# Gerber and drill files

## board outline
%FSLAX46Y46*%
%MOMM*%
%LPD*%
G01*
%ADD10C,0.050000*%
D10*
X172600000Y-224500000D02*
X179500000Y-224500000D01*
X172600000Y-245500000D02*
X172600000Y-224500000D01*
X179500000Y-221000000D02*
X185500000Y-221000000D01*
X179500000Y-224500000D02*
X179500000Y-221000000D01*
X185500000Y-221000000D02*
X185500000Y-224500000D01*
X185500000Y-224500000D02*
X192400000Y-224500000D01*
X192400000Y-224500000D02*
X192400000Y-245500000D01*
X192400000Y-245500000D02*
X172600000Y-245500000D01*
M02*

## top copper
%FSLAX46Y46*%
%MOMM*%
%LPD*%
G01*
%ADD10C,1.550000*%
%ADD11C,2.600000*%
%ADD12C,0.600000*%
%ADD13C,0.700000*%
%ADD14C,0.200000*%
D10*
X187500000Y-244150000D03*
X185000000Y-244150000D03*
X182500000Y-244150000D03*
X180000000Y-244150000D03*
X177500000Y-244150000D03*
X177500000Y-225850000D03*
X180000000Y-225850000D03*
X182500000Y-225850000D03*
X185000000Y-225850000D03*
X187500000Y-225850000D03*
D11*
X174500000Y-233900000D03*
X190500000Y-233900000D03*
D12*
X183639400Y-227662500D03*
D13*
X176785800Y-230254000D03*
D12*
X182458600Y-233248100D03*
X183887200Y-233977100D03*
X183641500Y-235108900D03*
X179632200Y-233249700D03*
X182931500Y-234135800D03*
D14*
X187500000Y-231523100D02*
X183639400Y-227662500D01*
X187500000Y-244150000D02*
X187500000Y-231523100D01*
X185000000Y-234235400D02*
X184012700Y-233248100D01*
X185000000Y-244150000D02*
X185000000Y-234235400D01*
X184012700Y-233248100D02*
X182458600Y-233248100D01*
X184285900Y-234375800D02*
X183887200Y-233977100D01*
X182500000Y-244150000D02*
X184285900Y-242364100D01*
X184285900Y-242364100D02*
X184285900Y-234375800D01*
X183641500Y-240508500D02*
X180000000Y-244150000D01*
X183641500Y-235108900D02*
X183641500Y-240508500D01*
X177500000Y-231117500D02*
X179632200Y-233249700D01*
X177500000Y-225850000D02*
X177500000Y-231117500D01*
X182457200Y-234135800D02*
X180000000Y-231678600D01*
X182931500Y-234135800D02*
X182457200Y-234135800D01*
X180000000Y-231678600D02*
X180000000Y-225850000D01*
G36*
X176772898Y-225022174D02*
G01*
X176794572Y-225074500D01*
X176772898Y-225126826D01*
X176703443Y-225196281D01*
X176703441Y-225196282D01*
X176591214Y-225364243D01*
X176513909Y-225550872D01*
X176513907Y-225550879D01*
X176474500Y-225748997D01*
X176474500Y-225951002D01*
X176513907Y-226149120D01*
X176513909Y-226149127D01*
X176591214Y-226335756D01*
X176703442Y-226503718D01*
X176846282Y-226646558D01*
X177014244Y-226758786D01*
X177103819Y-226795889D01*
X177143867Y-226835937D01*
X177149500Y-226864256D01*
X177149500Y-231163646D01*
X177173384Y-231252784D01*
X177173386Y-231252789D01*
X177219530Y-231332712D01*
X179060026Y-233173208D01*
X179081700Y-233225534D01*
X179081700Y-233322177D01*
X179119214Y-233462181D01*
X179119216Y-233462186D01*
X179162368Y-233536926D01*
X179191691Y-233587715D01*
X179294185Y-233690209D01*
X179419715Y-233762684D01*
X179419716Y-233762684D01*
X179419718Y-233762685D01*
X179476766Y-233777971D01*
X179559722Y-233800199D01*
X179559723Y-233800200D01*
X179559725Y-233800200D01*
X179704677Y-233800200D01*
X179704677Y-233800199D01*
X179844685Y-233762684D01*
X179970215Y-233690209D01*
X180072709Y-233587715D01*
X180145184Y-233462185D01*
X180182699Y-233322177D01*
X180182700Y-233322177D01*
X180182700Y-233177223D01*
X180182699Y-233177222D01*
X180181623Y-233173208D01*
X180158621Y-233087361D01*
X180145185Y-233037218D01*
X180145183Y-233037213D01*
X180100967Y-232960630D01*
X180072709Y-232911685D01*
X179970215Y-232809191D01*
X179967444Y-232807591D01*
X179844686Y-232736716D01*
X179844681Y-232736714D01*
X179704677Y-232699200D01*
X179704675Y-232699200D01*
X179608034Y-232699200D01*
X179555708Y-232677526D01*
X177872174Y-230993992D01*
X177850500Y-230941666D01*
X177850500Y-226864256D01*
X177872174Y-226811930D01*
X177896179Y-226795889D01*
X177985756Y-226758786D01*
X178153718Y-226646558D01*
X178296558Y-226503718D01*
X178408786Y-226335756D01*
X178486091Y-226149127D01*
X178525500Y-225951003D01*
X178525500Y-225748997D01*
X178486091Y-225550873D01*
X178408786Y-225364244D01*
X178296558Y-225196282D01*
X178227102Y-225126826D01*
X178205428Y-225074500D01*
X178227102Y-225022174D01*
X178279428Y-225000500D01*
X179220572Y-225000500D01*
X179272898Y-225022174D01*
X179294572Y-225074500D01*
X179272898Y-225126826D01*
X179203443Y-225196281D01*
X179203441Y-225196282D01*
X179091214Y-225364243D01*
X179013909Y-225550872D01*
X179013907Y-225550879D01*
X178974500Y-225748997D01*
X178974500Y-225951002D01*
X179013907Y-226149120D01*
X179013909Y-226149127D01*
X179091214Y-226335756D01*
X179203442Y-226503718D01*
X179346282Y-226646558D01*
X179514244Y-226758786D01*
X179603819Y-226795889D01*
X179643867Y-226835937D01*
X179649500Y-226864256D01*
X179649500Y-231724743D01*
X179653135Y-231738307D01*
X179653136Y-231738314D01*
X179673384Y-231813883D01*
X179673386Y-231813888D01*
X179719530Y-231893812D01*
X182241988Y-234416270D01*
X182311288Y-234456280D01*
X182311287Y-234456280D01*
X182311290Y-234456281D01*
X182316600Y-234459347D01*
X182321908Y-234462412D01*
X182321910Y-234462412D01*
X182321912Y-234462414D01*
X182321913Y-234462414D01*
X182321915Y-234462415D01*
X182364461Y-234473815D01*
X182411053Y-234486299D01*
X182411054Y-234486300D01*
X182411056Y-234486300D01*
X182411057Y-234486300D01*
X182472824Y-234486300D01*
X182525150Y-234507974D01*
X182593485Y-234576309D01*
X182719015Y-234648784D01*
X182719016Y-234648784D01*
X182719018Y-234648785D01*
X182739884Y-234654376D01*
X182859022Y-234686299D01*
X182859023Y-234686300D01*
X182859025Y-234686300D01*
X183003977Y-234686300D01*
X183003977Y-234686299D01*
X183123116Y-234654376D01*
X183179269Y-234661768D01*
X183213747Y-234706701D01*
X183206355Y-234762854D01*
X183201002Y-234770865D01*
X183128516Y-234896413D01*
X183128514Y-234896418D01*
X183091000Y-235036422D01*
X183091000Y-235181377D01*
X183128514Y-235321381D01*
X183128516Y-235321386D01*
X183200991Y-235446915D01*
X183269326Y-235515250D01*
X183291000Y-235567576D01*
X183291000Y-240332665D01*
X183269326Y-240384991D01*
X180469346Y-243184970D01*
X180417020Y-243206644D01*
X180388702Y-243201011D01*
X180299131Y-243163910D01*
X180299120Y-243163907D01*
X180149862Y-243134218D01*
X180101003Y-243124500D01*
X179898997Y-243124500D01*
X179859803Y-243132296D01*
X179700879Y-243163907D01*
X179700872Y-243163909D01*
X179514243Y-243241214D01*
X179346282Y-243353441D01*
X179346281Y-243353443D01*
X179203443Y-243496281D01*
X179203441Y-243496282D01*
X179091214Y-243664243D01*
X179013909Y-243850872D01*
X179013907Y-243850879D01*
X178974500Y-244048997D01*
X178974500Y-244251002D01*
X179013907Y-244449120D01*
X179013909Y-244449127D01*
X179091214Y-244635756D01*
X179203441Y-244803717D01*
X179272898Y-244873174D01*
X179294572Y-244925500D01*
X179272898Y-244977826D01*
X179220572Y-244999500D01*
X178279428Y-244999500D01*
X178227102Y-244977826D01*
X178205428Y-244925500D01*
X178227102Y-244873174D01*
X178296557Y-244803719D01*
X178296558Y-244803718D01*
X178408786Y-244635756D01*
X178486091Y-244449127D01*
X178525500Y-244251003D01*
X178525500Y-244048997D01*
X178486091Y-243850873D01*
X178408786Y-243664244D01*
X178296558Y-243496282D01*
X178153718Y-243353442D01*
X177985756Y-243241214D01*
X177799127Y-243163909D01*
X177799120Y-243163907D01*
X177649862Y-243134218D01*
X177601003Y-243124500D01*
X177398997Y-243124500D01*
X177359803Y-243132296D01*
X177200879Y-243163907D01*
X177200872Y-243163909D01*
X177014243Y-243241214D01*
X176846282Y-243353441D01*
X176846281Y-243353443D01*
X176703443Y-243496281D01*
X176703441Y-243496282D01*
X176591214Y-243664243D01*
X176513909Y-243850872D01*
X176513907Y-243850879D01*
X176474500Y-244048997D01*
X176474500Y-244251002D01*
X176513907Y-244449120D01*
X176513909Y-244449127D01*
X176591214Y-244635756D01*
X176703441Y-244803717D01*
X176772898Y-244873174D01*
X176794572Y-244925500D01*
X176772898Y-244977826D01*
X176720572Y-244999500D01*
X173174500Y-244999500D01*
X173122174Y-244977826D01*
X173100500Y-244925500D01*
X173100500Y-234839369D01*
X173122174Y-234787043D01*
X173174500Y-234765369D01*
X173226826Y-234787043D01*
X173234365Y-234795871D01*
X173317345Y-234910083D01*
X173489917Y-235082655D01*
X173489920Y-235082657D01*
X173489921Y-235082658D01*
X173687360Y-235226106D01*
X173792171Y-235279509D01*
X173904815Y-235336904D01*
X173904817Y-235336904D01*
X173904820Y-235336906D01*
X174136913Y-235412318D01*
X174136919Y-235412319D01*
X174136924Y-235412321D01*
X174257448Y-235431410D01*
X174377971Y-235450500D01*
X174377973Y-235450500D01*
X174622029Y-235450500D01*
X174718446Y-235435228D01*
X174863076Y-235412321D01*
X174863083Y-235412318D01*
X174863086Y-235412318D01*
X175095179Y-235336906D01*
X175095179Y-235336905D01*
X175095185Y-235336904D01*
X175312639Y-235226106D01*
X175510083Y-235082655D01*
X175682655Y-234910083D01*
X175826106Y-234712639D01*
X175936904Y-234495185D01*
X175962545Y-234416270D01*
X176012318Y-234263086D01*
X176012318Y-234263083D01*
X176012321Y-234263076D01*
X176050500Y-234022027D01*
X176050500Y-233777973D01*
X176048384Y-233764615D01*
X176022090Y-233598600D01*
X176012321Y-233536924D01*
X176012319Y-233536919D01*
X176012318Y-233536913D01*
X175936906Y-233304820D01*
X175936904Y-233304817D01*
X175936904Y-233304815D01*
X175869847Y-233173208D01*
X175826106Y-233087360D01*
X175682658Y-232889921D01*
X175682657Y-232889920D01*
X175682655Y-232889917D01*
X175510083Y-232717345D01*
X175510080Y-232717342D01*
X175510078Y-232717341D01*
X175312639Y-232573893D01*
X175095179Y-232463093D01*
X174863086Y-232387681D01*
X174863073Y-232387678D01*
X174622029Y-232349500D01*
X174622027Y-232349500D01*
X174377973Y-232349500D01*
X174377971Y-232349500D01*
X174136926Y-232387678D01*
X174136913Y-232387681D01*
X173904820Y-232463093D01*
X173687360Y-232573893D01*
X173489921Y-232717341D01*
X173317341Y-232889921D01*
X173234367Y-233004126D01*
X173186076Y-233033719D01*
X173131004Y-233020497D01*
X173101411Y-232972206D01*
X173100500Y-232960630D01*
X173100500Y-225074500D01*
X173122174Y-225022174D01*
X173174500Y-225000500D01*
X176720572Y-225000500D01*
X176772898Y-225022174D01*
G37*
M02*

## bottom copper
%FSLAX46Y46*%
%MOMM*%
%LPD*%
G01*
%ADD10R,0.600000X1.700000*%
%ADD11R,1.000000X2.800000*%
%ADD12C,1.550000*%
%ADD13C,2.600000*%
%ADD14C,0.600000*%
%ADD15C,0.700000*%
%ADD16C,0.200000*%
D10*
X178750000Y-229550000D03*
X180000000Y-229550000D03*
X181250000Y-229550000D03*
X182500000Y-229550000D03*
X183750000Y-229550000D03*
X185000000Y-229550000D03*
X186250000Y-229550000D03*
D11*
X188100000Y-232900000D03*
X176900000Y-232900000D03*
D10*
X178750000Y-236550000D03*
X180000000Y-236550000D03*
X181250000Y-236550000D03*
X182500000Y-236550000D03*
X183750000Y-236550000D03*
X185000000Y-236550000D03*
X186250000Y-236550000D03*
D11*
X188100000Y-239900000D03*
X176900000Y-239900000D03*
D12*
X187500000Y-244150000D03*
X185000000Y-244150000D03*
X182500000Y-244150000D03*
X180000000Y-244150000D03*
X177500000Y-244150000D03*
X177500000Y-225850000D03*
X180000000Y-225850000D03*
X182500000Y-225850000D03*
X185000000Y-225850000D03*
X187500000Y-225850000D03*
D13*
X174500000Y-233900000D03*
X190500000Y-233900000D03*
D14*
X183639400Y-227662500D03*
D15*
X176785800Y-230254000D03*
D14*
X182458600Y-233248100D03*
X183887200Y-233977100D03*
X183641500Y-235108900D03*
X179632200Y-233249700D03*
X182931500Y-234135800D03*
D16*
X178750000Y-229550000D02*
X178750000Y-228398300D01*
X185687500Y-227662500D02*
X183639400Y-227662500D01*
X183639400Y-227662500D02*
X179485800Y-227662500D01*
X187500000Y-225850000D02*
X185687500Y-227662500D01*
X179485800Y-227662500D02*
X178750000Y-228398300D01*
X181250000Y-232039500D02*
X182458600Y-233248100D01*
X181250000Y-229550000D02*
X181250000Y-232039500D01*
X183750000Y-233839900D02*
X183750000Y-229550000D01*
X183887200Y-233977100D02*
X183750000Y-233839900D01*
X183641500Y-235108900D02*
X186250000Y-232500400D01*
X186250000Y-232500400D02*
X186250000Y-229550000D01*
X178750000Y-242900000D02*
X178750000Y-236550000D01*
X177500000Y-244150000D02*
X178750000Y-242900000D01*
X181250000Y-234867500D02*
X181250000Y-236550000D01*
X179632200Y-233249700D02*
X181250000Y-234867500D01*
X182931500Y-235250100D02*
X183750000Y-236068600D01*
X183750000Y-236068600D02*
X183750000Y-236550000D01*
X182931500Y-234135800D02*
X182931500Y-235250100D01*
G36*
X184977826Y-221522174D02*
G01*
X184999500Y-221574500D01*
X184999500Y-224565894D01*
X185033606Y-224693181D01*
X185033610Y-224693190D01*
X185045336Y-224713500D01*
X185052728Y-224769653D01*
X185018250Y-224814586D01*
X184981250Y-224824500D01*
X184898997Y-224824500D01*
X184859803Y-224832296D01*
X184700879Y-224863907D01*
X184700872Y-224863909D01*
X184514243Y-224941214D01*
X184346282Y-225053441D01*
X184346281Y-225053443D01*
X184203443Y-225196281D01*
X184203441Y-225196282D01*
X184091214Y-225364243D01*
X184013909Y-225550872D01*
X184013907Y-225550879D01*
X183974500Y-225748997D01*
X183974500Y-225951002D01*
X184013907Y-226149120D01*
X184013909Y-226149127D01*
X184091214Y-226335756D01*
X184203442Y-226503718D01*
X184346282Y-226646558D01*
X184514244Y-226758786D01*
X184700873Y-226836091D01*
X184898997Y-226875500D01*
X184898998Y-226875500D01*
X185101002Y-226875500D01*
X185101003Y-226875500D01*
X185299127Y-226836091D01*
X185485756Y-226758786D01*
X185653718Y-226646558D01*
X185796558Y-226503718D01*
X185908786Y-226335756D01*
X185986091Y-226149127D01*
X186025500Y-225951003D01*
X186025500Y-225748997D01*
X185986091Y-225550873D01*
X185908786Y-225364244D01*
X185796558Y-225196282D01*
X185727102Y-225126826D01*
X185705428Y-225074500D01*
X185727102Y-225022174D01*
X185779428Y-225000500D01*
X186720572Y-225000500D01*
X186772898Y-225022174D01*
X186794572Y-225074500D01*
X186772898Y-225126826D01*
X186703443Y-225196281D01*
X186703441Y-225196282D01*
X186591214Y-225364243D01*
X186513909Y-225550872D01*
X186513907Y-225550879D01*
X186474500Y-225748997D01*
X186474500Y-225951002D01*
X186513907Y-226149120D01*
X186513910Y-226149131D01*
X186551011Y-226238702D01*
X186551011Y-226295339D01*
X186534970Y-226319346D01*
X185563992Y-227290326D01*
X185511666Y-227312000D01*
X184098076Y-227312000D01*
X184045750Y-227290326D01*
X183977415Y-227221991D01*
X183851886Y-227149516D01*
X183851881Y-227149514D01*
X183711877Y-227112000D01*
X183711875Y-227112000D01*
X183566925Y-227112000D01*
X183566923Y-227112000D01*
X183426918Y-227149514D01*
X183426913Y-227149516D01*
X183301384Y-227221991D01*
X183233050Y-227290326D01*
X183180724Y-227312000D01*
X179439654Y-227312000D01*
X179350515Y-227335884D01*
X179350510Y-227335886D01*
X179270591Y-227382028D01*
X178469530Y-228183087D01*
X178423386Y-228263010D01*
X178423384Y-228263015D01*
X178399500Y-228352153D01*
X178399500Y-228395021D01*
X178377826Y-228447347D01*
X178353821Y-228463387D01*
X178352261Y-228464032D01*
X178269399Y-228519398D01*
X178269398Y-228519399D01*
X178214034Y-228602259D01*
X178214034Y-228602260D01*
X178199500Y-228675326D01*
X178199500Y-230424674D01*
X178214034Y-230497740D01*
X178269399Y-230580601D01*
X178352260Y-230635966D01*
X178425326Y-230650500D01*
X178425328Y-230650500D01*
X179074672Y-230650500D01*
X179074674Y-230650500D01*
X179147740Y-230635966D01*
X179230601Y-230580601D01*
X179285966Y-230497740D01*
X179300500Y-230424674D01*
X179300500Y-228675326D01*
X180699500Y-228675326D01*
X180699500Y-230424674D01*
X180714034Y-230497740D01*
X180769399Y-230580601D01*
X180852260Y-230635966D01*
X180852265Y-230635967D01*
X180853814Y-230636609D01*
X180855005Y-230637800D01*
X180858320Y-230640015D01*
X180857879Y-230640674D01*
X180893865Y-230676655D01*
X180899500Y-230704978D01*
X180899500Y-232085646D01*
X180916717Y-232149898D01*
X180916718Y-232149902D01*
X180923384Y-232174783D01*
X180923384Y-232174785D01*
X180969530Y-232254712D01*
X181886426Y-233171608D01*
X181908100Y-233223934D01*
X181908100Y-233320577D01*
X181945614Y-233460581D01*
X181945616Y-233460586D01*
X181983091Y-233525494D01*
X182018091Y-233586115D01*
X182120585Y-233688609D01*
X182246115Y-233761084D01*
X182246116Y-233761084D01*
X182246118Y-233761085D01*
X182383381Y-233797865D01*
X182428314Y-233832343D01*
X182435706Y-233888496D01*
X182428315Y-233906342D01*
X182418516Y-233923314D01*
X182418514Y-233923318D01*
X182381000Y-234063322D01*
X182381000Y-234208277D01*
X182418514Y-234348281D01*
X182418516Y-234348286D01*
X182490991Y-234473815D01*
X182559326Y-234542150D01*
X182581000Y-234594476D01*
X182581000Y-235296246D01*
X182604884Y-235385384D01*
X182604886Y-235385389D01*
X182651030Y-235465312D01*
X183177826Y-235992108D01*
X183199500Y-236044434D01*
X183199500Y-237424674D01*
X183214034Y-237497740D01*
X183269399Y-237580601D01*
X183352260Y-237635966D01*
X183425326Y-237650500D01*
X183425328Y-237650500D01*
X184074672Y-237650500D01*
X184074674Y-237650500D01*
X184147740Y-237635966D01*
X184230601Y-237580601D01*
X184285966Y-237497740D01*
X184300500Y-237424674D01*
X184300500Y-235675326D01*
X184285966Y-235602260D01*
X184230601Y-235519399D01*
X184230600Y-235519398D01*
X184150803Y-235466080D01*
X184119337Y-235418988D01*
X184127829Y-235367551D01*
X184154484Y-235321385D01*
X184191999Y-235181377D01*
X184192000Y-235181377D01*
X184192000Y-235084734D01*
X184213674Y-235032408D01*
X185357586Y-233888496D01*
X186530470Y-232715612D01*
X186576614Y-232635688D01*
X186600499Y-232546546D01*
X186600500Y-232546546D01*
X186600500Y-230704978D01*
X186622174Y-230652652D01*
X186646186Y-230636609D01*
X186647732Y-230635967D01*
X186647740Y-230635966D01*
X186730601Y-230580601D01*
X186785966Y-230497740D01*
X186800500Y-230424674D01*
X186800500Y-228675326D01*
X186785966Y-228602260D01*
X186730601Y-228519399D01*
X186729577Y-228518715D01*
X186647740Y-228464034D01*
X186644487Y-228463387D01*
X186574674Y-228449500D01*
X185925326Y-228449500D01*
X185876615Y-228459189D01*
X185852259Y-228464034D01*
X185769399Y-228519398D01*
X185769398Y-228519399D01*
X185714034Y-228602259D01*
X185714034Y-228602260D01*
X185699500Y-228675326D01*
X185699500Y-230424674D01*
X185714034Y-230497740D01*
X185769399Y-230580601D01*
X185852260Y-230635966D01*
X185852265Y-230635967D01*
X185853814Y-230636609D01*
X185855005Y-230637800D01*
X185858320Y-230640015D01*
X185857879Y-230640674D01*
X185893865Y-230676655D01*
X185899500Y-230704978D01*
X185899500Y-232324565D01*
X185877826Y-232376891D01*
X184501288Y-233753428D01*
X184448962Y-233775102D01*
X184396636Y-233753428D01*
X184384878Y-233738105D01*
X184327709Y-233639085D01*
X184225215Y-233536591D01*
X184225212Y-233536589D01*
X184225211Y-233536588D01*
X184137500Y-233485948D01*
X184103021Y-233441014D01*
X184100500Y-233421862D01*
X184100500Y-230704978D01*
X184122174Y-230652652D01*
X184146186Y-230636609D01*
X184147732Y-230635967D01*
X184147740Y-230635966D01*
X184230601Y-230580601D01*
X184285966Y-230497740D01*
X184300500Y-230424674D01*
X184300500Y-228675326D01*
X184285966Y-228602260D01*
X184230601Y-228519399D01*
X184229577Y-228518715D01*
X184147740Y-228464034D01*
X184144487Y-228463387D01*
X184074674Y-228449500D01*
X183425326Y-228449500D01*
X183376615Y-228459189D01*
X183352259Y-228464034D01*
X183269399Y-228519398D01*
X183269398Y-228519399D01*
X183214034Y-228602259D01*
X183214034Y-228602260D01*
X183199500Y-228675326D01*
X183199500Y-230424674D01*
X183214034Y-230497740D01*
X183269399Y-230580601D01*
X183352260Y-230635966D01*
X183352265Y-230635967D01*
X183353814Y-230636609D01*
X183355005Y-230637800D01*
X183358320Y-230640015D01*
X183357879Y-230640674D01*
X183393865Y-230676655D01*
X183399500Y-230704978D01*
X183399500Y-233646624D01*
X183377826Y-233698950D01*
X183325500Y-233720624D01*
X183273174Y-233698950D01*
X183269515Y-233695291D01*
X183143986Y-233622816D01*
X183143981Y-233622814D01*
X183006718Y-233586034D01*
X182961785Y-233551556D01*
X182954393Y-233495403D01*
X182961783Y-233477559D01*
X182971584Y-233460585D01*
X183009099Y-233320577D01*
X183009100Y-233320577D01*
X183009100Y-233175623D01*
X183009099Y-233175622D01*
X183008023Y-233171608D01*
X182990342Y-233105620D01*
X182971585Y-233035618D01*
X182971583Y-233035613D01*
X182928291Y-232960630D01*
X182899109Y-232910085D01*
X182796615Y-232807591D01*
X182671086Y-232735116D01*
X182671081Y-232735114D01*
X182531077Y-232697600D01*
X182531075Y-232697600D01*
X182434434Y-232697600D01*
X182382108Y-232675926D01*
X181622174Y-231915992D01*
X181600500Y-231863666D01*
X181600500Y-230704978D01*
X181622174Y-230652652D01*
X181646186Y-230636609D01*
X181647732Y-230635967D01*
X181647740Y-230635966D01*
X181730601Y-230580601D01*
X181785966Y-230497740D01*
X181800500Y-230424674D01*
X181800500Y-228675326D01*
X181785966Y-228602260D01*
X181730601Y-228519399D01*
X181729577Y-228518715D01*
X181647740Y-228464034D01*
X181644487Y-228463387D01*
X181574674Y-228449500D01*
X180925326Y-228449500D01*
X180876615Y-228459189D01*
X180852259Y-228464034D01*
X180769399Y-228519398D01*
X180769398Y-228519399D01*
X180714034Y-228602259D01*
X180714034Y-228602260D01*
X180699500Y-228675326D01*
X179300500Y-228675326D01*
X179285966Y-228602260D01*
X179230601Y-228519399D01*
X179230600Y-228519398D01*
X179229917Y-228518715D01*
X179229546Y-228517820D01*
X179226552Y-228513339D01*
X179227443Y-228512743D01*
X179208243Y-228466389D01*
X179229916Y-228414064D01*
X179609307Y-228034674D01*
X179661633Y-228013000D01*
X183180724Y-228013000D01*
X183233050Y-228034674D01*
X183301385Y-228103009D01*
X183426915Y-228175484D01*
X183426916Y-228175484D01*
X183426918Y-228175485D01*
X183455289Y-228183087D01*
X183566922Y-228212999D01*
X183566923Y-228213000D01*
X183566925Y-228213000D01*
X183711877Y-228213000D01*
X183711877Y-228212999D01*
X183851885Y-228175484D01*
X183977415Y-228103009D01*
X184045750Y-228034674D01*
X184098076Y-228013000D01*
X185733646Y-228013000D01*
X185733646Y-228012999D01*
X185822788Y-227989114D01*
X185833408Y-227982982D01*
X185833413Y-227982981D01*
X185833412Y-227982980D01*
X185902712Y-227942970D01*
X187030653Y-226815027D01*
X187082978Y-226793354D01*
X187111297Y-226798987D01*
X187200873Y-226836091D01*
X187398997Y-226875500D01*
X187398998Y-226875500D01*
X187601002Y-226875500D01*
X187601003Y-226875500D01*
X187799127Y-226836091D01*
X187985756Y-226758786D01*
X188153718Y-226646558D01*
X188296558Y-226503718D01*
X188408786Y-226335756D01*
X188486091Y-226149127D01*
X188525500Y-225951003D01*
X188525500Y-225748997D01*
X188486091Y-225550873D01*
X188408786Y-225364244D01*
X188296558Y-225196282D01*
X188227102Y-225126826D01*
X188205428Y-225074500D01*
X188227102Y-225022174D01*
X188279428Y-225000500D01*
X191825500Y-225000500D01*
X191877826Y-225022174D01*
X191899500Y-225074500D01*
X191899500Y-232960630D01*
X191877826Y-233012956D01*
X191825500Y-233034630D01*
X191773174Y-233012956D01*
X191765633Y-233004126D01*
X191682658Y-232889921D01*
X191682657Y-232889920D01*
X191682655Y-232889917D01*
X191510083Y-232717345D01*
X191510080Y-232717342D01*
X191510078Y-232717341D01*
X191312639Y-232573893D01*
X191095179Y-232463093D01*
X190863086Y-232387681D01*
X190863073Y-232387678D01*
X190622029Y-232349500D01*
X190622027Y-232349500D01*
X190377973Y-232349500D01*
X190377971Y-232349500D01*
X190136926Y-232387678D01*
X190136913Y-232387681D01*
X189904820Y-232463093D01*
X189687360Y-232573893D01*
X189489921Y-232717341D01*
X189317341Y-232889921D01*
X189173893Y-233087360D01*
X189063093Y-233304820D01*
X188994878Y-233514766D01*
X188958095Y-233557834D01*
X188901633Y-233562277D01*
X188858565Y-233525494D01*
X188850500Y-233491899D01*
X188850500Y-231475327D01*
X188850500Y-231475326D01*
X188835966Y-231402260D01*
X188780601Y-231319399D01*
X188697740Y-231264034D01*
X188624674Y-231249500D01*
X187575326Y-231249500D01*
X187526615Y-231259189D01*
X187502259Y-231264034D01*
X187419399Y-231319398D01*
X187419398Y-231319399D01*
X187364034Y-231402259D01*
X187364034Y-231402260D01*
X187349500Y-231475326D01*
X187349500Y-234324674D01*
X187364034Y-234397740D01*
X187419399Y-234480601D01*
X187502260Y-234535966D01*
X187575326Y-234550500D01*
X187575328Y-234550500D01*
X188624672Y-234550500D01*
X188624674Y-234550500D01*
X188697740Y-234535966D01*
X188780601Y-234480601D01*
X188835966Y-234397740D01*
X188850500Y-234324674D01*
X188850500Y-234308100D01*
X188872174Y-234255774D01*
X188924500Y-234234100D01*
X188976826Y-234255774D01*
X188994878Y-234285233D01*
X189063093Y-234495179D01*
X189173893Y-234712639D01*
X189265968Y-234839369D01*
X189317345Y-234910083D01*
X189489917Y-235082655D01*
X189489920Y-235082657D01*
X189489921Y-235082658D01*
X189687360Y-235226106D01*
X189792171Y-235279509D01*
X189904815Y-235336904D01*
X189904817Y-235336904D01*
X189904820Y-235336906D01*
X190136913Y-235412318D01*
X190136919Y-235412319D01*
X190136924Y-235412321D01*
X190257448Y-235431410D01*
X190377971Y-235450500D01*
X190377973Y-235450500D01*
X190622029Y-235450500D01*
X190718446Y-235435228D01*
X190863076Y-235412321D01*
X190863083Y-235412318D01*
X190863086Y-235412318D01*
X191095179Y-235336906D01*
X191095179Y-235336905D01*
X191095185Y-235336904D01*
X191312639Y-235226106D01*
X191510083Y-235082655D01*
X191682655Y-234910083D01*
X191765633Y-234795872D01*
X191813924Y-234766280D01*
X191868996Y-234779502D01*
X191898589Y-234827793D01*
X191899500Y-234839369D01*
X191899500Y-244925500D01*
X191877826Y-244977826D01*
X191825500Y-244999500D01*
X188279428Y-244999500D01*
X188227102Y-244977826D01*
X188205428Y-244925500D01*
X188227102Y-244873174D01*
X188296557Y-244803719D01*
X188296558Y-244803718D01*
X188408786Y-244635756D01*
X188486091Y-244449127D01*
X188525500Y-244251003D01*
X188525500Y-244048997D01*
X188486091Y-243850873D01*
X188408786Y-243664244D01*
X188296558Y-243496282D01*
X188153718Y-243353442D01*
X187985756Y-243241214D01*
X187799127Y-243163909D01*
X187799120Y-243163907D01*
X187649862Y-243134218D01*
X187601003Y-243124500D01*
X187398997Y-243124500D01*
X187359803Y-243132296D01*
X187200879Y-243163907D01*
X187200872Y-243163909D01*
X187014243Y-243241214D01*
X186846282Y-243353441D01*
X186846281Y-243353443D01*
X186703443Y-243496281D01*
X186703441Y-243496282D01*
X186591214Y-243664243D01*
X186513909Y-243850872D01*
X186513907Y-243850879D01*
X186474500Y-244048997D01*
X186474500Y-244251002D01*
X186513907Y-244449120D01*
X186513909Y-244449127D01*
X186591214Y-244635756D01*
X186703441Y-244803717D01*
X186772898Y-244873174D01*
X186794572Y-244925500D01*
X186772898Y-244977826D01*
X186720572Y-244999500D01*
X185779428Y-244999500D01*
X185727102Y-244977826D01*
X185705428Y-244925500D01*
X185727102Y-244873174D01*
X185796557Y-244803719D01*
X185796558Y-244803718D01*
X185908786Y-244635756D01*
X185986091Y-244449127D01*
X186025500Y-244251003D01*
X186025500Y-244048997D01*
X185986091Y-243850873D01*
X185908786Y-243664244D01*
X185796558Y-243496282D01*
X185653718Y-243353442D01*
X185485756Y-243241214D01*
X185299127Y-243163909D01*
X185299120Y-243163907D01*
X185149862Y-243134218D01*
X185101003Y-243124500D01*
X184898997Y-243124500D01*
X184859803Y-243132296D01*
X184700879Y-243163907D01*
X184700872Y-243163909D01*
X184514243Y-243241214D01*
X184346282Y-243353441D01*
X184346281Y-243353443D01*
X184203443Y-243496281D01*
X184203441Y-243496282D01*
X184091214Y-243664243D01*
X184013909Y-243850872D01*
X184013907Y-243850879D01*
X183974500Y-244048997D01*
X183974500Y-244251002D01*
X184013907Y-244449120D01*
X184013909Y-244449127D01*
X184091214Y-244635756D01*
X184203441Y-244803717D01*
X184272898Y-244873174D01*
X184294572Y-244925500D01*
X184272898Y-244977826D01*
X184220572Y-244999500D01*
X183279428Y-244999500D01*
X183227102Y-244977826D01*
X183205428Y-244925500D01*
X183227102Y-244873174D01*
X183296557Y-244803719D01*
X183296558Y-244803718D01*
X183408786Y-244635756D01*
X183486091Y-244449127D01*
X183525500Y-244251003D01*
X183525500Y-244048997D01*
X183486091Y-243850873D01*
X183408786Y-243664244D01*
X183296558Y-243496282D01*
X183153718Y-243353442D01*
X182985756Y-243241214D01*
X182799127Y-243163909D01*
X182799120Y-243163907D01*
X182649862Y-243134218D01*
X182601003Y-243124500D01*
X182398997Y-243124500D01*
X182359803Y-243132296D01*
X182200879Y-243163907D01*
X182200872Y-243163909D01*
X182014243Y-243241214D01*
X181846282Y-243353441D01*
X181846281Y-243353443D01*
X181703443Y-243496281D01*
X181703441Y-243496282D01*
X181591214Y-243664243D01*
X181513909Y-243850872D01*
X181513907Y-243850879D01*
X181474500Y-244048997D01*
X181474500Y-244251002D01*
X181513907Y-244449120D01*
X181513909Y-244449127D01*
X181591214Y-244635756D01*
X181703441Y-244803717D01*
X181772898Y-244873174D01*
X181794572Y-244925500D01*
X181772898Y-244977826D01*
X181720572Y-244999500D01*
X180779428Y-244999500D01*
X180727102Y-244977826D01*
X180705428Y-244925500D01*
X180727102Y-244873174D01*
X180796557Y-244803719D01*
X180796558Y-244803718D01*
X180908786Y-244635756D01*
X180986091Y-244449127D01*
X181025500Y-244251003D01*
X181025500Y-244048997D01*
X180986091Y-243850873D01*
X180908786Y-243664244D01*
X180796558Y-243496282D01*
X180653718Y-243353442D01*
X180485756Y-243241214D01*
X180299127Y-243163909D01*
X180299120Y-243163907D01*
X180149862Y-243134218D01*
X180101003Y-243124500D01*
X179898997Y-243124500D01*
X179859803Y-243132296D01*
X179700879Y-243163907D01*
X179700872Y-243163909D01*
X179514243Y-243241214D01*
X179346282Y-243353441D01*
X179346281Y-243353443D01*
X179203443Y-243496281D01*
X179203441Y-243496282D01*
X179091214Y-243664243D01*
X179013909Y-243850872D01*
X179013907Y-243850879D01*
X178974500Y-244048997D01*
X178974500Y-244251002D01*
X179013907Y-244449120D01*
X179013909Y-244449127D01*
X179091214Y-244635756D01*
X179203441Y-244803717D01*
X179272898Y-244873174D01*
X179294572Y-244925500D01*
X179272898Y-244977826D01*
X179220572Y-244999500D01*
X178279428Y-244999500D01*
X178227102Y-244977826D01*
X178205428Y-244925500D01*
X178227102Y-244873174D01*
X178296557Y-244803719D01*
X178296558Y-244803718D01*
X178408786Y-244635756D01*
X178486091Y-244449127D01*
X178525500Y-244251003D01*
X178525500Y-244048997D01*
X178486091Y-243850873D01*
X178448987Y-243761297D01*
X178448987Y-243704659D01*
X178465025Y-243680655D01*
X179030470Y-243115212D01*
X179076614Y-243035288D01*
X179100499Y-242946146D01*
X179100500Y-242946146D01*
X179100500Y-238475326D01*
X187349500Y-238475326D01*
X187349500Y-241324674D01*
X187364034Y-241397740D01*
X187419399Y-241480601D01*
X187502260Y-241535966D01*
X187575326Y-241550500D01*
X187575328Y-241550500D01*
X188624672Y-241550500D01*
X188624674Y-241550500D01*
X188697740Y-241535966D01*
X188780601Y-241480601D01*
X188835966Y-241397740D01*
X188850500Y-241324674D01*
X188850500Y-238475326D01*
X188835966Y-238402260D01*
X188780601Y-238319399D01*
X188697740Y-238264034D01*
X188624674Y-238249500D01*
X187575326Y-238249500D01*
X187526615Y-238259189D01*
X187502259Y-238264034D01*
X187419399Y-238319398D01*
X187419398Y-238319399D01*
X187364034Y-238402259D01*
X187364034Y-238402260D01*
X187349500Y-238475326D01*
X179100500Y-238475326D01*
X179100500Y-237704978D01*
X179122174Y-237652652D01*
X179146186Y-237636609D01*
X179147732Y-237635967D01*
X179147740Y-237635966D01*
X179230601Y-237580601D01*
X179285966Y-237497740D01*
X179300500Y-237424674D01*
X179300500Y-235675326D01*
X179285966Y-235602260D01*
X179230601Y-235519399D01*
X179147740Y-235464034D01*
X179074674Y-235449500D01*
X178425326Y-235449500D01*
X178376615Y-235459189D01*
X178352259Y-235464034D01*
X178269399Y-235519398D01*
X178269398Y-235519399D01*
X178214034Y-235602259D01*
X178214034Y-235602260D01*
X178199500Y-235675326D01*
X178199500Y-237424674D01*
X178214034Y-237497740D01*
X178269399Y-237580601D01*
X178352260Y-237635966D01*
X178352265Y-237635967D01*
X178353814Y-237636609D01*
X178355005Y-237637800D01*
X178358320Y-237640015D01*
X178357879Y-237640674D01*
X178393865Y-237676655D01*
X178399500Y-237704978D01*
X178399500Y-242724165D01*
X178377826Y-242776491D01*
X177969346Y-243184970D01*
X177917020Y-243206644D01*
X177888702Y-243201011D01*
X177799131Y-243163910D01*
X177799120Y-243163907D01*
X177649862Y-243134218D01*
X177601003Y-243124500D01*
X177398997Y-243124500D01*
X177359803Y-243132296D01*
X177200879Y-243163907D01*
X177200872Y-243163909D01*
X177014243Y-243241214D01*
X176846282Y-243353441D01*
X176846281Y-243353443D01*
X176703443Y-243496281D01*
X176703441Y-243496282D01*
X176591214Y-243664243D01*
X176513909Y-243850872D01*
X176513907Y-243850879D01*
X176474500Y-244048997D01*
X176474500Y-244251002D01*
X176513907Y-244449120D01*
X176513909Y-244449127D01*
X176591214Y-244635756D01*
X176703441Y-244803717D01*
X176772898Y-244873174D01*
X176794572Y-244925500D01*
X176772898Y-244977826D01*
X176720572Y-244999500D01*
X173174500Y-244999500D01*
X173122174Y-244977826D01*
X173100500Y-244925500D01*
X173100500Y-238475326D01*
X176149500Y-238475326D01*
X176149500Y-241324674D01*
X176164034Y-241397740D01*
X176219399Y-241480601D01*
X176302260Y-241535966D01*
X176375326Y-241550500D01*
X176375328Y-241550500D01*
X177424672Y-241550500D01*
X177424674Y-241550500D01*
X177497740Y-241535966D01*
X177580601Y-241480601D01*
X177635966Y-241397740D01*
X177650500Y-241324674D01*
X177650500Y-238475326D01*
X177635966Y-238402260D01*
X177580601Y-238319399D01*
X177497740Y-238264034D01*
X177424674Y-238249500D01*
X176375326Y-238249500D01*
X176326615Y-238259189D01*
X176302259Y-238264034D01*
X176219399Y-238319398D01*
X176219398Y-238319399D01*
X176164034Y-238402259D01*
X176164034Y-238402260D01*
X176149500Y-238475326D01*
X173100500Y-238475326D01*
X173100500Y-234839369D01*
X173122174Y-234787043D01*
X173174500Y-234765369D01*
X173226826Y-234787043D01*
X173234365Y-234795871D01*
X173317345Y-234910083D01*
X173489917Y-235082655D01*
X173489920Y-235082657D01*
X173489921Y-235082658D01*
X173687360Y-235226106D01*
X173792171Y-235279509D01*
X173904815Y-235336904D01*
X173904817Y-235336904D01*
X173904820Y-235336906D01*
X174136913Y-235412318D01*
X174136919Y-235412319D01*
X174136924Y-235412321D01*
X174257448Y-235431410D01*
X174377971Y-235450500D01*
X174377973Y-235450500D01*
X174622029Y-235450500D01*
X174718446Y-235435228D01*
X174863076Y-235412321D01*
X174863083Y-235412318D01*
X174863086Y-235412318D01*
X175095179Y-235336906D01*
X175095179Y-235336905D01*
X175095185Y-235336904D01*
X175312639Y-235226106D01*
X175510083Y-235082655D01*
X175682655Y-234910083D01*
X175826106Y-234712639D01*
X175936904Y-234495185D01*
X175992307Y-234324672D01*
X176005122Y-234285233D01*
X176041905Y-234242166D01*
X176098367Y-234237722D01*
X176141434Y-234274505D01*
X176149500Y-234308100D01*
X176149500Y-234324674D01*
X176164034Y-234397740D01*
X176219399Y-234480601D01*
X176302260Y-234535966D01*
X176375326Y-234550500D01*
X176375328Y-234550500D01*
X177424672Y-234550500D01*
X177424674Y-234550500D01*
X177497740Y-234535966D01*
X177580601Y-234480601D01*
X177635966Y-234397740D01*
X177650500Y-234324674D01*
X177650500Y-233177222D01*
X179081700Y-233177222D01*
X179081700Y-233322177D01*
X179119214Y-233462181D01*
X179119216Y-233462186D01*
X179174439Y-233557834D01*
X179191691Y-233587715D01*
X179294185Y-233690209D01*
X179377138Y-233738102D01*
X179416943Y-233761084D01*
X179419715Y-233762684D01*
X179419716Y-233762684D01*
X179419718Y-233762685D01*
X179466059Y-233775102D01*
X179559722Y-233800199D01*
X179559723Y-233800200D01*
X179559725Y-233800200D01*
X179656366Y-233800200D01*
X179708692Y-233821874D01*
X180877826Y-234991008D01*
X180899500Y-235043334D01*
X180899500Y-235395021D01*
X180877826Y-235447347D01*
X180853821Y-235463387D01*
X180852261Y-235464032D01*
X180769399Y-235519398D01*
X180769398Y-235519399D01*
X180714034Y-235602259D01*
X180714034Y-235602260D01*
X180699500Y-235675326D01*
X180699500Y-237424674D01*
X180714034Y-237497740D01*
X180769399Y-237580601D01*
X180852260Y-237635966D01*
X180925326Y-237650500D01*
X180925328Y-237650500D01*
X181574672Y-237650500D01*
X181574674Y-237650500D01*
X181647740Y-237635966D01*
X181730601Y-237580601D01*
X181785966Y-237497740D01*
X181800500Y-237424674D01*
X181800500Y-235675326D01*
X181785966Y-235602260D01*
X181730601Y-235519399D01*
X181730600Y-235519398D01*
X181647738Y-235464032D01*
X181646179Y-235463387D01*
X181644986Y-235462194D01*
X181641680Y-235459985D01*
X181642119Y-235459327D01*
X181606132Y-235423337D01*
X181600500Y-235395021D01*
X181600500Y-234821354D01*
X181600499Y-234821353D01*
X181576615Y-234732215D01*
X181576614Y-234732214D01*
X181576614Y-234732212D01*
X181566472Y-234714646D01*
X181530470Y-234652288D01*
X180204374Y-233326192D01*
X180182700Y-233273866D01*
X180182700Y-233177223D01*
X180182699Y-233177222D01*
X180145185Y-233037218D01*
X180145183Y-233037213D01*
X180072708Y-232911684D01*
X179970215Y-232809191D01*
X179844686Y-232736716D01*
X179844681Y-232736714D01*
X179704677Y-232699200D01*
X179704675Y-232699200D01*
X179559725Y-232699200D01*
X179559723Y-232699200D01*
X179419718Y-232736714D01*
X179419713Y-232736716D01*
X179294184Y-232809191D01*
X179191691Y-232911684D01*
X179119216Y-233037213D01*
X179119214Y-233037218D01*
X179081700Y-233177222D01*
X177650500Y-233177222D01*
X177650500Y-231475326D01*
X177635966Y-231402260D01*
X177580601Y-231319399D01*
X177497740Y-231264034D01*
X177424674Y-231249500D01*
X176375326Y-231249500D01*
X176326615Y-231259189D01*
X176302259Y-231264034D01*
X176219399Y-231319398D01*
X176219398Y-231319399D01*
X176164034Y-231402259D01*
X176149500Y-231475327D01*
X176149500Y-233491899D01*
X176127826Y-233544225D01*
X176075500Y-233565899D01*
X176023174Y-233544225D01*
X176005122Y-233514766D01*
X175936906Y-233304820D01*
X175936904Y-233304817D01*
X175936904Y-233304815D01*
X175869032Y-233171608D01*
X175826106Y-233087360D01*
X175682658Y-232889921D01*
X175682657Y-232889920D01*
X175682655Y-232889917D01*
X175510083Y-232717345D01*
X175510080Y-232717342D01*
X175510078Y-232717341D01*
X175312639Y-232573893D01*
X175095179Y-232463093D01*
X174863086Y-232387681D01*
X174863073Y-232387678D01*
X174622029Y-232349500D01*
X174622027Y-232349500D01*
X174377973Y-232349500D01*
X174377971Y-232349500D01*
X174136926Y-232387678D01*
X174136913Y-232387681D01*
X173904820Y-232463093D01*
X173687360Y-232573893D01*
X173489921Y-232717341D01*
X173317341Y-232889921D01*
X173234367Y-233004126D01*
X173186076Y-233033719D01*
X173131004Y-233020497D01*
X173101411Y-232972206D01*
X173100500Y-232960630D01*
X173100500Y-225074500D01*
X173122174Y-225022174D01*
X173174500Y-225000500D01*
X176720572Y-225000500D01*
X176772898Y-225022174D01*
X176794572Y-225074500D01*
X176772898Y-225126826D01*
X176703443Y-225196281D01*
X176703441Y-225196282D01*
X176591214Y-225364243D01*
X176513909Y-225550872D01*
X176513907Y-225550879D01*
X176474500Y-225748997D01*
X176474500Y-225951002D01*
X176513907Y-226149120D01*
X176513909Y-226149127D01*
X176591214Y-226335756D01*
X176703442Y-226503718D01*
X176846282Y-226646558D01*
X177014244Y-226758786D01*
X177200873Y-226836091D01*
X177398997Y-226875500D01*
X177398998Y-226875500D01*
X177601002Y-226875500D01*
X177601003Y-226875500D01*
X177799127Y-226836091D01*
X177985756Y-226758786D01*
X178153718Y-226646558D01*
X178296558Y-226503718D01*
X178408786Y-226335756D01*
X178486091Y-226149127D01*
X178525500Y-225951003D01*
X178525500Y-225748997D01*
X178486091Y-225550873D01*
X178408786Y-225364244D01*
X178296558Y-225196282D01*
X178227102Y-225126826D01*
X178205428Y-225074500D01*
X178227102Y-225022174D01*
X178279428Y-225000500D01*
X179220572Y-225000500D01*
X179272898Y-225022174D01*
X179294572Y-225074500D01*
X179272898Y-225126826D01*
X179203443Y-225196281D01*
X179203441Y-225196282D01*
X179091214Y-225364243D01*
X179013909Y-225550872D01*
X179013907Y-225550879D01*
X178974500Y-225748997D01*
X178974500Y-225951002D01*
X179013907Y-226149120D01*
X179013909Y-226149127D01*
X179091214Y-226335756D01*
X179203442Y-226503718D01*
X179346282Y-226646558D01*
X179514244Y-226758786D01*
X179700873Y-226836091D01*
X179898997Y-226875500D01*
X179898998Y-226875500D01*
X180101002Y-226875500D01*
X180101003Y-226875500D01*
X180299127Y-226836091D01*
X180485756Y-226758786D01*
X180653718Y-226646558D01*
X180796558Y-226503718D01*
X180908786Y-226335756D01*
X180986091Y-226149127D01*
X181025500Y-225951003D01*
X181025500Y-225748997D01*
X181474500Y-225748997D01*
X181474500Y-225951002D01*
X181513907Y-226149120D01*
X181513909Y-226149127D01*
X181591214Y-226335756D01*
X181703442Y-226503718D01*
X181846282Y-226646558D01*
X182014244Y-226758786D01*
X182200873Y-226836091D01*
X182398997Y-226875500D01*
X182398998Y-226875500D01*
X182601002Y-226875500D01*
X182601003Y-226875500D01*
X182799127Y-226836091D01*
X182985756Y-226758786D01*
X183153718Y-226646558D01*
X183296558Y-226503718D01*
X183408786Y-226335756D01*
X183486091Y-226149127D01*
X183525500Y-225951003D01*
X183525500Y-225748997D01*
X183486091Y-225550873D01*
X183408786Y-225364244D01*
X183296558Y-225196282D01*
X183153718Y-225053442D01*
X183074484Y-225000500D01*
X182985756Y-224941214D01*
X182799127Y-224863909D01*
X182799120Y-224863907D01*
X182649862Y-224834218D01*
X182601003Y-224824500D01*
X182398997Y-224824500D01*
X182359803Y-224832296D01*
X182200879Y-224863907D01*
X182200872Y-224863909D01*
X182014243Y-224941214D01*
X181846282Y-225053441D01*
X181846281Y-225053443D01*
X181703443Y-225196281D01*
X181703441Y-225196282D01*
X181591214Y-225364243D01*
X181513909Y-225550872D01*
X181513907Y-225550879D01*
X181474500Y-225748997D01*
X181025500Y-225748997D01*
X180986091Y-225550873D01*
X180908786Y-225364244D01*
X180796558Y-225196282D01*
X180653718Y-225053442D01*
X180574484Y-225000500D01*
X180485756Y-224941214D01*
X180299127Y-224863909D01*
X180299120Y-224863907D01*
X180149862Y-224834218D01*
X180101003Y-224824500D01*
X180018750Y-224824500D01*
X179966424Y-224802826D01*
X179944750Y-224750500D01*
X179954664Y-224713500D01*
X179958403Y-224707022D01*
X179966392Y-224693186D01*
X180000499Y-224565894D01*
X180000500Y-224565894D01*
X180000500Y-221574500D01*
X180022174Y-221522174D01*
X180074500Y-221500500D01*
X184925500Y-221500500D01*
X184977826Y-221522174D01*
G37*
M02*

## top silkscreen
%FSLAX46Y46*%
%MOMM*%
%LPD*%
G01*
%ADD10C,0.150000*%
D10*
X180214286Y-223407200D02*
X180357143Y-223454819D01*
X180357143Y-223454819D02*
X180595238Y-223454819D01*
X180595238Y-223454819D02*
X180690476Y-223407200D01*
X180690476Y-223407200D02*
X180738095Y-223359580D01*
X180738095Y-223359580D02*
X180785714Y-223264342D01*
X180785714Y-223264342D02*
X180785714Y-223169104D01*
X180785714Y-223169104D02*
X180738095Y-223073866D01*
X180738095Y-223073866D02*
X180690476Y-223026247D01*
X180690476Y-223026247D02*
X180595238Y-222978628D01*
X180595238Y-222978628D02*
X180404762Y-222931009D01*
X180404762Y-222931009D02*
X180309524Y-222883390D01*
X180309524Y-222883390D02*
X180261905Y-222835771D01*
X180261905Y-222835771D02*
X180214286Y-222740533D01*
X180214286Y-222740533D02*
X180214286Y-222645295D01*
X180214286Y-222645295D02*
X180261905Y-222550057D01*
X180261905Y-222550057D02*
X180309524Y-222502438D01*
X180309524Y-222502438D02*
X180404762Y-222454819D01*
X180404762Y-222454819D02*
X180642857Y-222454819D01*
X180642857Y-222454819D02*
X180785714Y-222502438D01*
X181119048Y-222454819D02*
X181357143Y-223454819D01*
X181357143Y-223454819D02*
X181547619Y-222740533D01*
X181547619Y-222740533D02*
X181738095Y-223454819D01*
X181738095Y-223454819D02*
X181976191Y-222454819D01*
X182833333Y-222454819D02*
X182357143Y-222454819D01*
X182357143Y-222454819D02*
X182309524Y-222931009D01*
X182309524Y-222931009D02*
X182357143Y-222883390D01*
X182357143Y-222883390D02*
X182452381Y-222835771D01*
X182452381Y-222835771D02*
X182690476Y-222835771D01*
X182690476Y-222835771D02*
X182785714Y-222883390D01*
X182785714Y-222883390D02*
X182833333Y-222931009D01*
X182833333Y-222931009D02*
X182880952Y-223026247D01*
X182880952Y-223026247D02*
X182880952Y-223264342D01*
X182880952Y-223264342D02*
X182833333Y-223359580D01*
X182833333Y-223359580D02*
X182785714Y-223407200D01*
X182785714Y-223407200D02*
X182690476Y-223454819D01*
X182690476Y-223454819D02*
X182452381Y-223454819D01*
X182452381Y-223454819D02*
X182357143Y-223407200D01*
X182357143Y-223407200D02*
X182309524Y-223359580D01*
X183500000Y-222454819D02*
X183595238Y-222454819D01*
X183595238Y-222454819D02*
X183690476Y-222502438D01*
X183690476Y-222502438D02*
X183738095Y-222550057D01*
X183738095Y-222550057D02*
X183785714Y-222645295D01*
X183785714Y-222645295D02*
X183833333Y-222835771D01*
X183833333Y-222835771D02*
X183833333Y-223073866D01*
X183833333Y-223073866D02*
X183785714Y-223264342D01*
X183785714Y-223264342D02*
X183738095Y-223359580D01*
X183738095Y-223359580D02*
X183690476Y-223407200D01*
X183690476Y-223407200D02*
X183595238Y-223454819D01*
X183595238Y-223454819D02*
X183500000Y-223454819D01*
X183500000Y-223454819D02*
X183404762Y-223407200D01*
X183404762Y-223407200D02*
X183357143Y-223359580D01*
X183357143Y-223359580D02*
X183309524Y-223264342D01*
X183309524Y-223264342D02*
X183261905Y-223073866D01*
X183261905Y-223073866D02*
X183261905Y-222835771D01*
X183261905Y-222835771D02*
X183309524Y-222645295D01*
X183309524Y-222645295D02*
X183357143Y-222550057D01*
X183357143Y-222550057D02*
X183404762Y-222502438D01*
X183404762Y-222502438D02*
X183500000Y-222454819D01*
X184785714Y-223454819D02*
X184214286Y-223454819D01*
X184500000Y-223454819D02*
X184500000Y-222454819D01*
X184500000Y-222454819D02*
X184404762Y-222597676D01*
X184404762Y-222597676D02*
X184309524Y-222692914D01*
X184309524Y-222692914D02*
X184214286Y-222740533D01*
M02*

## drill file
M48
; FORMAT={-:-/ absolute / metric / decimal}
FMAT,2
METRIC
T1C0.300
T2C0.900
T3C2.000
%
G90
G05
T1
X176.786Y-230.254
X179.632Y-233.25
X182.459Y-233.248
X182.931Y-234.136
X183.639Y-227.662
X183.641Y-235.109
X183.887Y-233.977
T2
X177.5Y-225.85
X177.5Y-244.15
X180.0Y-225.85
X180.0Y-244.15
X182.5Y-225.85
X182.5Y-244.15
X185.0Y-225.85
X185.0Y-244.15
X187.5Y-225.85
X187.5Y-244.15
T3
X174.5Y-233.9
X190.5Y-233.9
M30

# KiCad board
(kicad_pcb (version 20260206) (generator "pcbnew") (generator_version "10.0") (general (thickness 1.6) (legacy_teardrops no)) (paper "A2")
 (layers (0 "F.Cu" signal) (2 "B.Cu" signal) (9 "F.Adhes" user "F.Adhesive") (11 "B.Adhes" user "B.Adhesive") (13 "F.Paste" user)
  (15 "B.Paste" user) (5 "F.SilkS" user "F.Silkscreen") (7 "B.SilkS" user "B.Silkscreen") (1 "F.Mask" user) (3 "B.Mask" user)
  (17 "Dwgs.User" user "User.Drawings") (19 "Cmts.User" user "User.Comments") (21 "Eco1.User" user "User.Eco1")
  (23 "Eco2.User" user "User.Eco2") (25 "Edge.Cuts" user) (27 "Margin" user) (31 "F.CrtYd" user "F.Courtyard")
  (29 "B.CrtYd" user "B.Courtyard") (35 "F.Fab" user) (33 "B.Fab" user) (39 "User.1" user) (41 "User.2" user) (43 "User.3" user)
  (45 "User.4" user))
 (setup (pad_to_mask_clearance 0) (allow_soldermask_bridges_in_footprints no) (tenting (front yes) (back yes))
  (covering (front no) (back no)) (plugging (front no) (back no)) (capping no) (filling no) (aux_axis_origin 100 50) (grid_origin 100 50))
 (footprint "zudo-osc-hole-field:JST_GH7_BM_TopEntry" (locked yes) (layer "B.Cu") (at 182.5 229.55 180)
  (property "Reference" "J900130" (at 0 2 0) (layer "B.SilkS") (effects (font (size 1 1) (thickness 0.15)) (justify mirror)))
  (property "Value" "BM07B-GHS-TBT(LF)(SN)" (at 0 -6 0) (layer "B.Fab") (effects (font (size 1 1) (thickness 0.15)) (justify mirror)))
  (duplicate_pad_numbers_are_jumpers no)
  (pad "1" smd rect (at 3.75 0 180) (size 0.6 1.7) (layers "B.Cu" "B.Mask" "B.Paste") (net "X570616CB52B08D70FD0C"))
  (pad "2" smd rect (at 2.5 0 180) (size 0.6 1.7) (layers "B.Cu" "B.Mask" "B.Paste") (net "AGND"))
  (pad "3" smd rect (at 1.25 0 180) (size 0.6 1.7) (layers "B.Cu" "B.Mask" "B.Paste") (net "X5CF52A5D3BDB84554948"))
  (pad "4" smd rect (at 0 0 180) (size 0.6 1.7) (layers "B.Cu" "B.Mask" "B.Paste") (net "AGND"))
  (pad "5" smd rect (at -1.25 0 180) (size 0.6 1.7) (layers "B.Cu" "B.Mask" "B.Paste") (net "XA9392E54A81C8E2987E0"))
  (pad "6" smd rect (at -2.5 0 180) (size 0.6 1.7) (layers "B.Cu" "B.Mask" "B.Paste") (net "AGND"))
  (pad "7" smd rect (at -3.75 0 180) (size 0.6 1.7) (layers "B.Cu" "B.Mask" "B.Paste") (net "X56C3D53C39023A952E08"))
  (pad "MP1" smd rect (at -5.6 -3.35 180) (size 1 2.8) (layers "B.Cu" "B.Mask" "B.Paste") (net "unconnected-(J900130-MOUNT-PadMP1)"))
  (pad "MP2" smd rect (at 5.6 -3.35 180) (size 1 2.8) (layers "B.Cu" "B.Mask" "B.Paste") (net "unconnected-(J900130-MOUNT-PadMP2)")))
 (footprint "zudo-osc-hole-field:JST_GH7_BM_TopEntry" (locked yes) (layer "B.Cu") (at 182.5 236.55 180)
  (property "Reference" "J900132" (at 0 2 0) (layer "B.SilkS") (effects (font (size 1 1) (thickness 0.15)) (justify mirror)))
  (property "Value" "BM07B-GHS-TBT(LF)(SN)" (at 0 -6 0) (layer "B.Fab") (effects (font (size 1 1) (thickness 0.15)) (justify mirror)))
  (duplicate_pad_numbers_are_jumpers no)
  (pad "1" smd rect (at 3.75 0 180) (size 0.6 1.7) (layers "B.Cu" "B.Mask" "B.Paste") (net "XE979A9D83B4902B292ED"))
  (pad "2" smd rect (at 2.5 0 180) (size 0.6 1.7) (layers "B.Cu" "B.Mask" "B.Paste") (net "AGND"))
  (pad "3" smd rect (at 1.25 0 180) (size 0.6 1.7) (layers "B.Cu" "B.Mask" "B.Paste") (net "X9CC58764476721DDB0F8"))
  (pad "4" smd rect (at 0 0 180) (size 0.6 1.7) (layers "B.Cu" "B.Mask" "B.Paste") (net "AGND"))
  (pad "5" smd rect (at -1.25 0 180) (size 0.6 1.7) (layers "B.Cu" "B.Mask" "B.Paste") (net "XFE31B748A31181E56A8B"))
  (pad "6" smd rect (at -2.5 0 180) (size 0.6 1.7) (layers "B.Cu" "B.Mask" "B.Paste") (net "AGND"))
  (pad "7" smd rect (at -3.75 0 180) (size 0.6 1.7) (layers "B.Cu" "B.Mask" "B.Paste") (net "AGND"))
  (pad "MP1" smd rect (at -5.6 -3.35 180) (size 1 2.8) (layers "B.Cu" "B.Mask" "B.Paste") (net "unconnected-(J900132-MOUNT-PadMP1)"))
  (pad "MP2" smd rect (at 5.6 -3.35 180) (size 1 2.8) (layers "B.Cu" "B.Mask" "B.Paste") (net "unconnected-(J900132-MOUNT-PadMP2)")))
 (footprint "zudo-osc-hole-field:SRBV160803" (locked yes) (layer "F.Cu") (at 182.5 235)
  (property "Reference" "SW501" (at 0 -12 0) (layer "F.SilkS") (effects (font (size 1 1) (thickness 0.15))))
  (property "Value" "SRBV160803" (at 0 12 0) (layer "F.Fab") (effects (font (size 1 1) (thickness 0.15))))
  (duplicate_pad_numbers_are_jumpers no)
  (pad "1" thru_hole circle (at 5 9.15) (size 1.55 1.55) (drill 0.9) (layers "*.Cu" "*.Mask") (remove_unused_layers no)
   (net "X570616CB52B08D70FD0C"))
  (pad "2" thru_hole circle (at 2.5 9.15) (size 1.55 1.55) (drill 0.9) (layers "*.Cu" "*.Mask") (remove_unused_layers no)
   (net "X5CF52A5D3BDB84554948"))
  (pad "3" thru_hole circle (at 0 9.15) (size 1.55 1.55) (drill 0.9) (layers "*.Cu" "*.Mask") (remove_unused_layers no)
   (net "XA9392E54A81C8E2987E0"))
  (pad "4" thru_hole circle (at -2.5 9.15) (size 1.55 1.55) (drill 0.9) (layers "*.Cu" "*.Mask") (remove_unused_layers no)
   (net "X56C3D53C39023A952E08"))
  (pad "5" thru_hole circle (at -5 9.15) (size 1.55 1.55) (drill 0.9) (layers "*.Cu" "*.Mask") (remove_unused_layers no)
   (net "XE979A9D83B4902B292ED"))
  (pad "6" thru_hole circle (at -5 -9.15) (size 1.55 1.55) (drill 0.9) (layers "*.Cu" "*.Mask") (remove_unused_layers no)
   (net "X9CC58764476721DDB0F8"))
  (pad "7" thru_hole circle (at -2.5 -9.15) (size 1.55 1.55) (drill 0.9) (layers "*.Cu" "*.Mask") (remove_unused_layers no)
   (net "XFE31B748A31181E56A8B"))
  (pad "8" thru_hole circle (at 0 -9.15) (size 1.55 1.55) (drill 0.9) (layers "*.Cu" "*.Mask") (remove_unused_layers no)
   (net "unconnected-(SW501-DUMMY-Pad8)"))
  (pad "9" thru_hole circle (at 2.5 -9.15) (size 1.55 1.55) (drill 0.9) (layers "*.Cu" "*.Mask") (remove_unused_layers no)
   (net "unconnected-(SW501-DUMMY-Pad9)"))
  (pad "10" thru_hole circle (at 5 -9.15) (size 1.55 1.55) (drill 0.9) (layers "*.Cu" "*.Mask") (remove_unused_layers no)
   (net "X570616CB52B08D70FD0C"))
  (pad "MP1" thru_hole circle (at -8 -1.1) (size 2.6 2.6) (drill 2) (layers "*.Cu" "*.Mask") (remove_unused_layers no)
   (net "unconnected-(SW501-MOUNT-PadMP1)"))
  (pad "MP2" thru_hole circle (at 8 -1.1) (size 2.6 2.6) (drill 2) (layers "*.Cu" "*.Mask") (remove_unused_layers no)
   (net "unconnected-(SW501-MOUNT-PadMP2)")))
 (gr_line (start 172.6 224.5) (end 179.5 224.5) (stroke (width 0.05) (type default)) (layer "Edge.Cuts"))
 (gr_line (start 172.6 245.5) (end 172.6 224.5) (stroke (width 0.05) (type default)) (layer "Edge.Cuts"))
 (gr_line (start 179.5 221) (end 185.5 221) (stroke (width 0.05) (type default)) (layer "Edge.Cuts"))
 (gr_line (start 179.5 224.5) (end 179.5 221) (stroke (width 0.05) (type default)) (layer "Edge.Cuts"))
 (gr_line (start 185.5 221) (end 185.5 224.5) (stroke (width 0.05) (type default)) (layer "Edge.Cuts"))
 (gr_line (start 185.5 224.5) (end 192.4 224.5) (stroke (width 0.05) (type default)) (layer "Edge.Cuts"))
 (gr_line (start 192.4 224.5) (end 192.4 245.5) (stroke (width 0.05) (type default)) (layer "Edge.Cuts"))
 (gr_line (start 192.4 245.5) (end 172.6 245.5) (stroke (width 0.05) (type default)) (layer "Edge.Cuts"))
 (segment (start 187.5 231.5231) (end 183.6394 227.6625) (width 0.2) (layer "F.Cu") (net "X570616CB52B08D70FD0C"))
 (segment (start 187.5 244.15) (end 187.5 231.5231) (width 0.2) (layer "F.Cu") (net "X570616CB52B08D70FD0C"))
 (via (at 183.6394 227.6625) (size 0.6) (drill 0.3) (layers "F.Cu" "B.Cu") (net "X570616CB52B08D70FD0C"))
 (segment (start 178.75 229.55) (end 178.75 228.3983) (width 0.2) (layer "B.Cu") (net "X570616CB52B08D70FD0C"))
 (segment (start 185.6875 227.6625) (end 183.6394 227.6625) (width 0.2) (layer "B.Cu") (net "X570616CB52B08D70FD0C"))
 (segment (start 183.6394 227.6625) (end 179.4858 227.6625) (width 0.2) (layer "B.Cu") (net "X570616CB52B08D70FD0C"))
 (segment (start 187.5 225.85) (end 185.6875 227.6625) (width 0.2) (layer "B.Cu") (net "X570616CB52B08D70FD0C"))
 (segment (start 179.4858 227.6625) (end 178.75 228.3983) (width 0.2) (layer "B.Cu") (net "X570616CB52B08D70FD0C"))
 (via (at 176.7858 230.254) (size 0.7) (drill 0.3) (layers "F.Cu" "B.Cu") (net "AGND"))
 (segment (start 185 234.2354) (end 184.0127 233.2481) (width 0.2) (layer "F.Cu") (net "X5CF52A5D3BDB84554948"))
 (segment (start 185 244.15) (end 185 234.2354) (width 0.2) (layer "F.Cu") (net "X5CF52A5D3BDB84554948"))
 (segment (start 184.0127 233.2481) (end 182.4586 233.2481) (width 0.2) (layer "F.Cu") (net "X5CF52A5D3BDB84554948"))
 (via (at 182.4586 233.2481) (size 0.6) (drill 0.3) (layers "F.Cu" "B.Cu") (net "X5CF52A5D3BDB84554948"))
 (segment (start 181.25 232.0395) (end 182.4586 233.2481) (width 0.2) (layer "B.Cu") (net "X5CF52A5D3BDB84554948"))
 (segment (start 181.25 229.55) (end 181.25 232.0395) (width 0.2) (layer "B.Cu") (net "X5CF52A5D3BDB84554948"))
 (segment (start 184.2859 234.3758) (end 183.8872 233.9771) (width 0.2) (layer "F.Cu") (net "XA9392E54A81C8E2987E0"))
 (segment (start 182.5 244.15) (end 184.2859 242.3641) (width 0.2) (layer "F.Cu") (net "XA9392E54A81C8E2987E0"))
 (segment (start 184.2859 242.3641) (end 184.2859 234.3758) (width 0.2) (layer "F.Cu") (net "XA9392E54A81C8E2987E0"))
 (via (at 183.8872 233.9771) (size 0.6) (drill 0.3) (layers "F.Cu" "B.Cu") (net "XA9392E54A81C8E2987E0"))
 (segment (start 183.75 233.8399) (end 183.75 229.55) (width 0.2) (layer "B.Cu") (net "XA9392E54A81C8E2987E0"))
 (segment (start 183.8872 233.9771) (end 183.75 233.8399) (width 0.2) (layer "B.Cu") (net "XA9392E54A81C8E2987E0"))
 (segment (start 183.6415 240.5085) (end 180 244.15) (width 0.2) (layer "F.Cu") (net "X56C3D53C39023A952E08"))
 (segment (start 183.6415 235.1089) (end 183.6415 240.5085) (width 0.2) (layer "F.Cu") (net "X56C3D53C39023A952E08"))
 (via (at 183.6415 235.1089) (size 0.6) (drill 0.3) (layers "F.Cu" "B.Cu") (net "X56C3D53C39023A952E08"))
 (segment (start 183.6415 235.1089) (end 186.25 232.5004) (width 0.2) (layer "B.Cu") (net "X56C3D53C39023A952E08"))
 (segment (start 186.25 232.5004) (end 186.25 229.55) (width 0.2) (layer "B.Cu") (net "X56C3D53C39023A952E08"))
 (segment (start 178.75 242.9) (end 178.75 236.55) (width 0.2) (layer "B.Cu") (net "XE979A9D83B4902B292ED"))
 (segment (start 177.5 244.15) (end 178.75 242.9) (width 0.2) (layer "B.Cu") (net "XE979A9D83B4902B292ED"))
 (segment (start 177.5 231.1175) (end 179.6322 233.2497) (width 0.2) (layer "F.Cu") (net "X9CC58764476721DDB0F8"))
 (segment (start 177.5 225.85) (end 177.5 231.1175) (width 0.2) (layer "F.Cu") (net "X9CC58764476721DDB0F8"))
 (via (at 179.6322 233.2497) (size 0.6) (drill 0.3) (layers "F.Cu" "B.Cu") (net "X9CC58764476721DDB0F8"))
 (segment (start 181.25 234.8675) (end 181.25 236.55) (width 0.2) (layer "B.Cu") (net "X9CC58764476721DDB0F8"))
 (segment (start 179.6322 233.2497) (end 181.25 234.8675) (width 0.2) (layer "B.Cu") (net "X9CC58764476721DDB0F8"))
 (segment (start 182.4572 234.1358) (end 180 231.6786) (width 0.2) (layer "F.Cu") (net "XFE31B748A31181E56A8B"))
 (segment (start 182.9315 234.1358) (end 182.4572 234.1358) (width 0.2) (layer "F.Cu") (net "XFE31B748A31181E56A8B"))
 (segment (start 180 231.6786) (end 180 225.85) (width 0.2) (layer "F.Cu") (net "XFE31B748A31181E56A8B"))
 (via (at 182.9315 234.1358) (size 0.6) (drill 0.3) (layers "F.Cu" "B.Cu") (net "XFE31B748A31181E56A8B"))
 (segment (start 182.9315 235.2501) (end 183.75 236.0686) (width 0.2) (layer "B.Cu") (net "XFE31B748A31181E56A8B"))
 (segment (start 183.75 236.0686) (end 183.75 236.55) (width 0.2) (layer "B.Cu") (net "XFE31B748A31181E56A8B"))
 (segment (start 182.9315 234.1358) (end 182.9315 235.2501) (width 0.2) (layer "B.Cu") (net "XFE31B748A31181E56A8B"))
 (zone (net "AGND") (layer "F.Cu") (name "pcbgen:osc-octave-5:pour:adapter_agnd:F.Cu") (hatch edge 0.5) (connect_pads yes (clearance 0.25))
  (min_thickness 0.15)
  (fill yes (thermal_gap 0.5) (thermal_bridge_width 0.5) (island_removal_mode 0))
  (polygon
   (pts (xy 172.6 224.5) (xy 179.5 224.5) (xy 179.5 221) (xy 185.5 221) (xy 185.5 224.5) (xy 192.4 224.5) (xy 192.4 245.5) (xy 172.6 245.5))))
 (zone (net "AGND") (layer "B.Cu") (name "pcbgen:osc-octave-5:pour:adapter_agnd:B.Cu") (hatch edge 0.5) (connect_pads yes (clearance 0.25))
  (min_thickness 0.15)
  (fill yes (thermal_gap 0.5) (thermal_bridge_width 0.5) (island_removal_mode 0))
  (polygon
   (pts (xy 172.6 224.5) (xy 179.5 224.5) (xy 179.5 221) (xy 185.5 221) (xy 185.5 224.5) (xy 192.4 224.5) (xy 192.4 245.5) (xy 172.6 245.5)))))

